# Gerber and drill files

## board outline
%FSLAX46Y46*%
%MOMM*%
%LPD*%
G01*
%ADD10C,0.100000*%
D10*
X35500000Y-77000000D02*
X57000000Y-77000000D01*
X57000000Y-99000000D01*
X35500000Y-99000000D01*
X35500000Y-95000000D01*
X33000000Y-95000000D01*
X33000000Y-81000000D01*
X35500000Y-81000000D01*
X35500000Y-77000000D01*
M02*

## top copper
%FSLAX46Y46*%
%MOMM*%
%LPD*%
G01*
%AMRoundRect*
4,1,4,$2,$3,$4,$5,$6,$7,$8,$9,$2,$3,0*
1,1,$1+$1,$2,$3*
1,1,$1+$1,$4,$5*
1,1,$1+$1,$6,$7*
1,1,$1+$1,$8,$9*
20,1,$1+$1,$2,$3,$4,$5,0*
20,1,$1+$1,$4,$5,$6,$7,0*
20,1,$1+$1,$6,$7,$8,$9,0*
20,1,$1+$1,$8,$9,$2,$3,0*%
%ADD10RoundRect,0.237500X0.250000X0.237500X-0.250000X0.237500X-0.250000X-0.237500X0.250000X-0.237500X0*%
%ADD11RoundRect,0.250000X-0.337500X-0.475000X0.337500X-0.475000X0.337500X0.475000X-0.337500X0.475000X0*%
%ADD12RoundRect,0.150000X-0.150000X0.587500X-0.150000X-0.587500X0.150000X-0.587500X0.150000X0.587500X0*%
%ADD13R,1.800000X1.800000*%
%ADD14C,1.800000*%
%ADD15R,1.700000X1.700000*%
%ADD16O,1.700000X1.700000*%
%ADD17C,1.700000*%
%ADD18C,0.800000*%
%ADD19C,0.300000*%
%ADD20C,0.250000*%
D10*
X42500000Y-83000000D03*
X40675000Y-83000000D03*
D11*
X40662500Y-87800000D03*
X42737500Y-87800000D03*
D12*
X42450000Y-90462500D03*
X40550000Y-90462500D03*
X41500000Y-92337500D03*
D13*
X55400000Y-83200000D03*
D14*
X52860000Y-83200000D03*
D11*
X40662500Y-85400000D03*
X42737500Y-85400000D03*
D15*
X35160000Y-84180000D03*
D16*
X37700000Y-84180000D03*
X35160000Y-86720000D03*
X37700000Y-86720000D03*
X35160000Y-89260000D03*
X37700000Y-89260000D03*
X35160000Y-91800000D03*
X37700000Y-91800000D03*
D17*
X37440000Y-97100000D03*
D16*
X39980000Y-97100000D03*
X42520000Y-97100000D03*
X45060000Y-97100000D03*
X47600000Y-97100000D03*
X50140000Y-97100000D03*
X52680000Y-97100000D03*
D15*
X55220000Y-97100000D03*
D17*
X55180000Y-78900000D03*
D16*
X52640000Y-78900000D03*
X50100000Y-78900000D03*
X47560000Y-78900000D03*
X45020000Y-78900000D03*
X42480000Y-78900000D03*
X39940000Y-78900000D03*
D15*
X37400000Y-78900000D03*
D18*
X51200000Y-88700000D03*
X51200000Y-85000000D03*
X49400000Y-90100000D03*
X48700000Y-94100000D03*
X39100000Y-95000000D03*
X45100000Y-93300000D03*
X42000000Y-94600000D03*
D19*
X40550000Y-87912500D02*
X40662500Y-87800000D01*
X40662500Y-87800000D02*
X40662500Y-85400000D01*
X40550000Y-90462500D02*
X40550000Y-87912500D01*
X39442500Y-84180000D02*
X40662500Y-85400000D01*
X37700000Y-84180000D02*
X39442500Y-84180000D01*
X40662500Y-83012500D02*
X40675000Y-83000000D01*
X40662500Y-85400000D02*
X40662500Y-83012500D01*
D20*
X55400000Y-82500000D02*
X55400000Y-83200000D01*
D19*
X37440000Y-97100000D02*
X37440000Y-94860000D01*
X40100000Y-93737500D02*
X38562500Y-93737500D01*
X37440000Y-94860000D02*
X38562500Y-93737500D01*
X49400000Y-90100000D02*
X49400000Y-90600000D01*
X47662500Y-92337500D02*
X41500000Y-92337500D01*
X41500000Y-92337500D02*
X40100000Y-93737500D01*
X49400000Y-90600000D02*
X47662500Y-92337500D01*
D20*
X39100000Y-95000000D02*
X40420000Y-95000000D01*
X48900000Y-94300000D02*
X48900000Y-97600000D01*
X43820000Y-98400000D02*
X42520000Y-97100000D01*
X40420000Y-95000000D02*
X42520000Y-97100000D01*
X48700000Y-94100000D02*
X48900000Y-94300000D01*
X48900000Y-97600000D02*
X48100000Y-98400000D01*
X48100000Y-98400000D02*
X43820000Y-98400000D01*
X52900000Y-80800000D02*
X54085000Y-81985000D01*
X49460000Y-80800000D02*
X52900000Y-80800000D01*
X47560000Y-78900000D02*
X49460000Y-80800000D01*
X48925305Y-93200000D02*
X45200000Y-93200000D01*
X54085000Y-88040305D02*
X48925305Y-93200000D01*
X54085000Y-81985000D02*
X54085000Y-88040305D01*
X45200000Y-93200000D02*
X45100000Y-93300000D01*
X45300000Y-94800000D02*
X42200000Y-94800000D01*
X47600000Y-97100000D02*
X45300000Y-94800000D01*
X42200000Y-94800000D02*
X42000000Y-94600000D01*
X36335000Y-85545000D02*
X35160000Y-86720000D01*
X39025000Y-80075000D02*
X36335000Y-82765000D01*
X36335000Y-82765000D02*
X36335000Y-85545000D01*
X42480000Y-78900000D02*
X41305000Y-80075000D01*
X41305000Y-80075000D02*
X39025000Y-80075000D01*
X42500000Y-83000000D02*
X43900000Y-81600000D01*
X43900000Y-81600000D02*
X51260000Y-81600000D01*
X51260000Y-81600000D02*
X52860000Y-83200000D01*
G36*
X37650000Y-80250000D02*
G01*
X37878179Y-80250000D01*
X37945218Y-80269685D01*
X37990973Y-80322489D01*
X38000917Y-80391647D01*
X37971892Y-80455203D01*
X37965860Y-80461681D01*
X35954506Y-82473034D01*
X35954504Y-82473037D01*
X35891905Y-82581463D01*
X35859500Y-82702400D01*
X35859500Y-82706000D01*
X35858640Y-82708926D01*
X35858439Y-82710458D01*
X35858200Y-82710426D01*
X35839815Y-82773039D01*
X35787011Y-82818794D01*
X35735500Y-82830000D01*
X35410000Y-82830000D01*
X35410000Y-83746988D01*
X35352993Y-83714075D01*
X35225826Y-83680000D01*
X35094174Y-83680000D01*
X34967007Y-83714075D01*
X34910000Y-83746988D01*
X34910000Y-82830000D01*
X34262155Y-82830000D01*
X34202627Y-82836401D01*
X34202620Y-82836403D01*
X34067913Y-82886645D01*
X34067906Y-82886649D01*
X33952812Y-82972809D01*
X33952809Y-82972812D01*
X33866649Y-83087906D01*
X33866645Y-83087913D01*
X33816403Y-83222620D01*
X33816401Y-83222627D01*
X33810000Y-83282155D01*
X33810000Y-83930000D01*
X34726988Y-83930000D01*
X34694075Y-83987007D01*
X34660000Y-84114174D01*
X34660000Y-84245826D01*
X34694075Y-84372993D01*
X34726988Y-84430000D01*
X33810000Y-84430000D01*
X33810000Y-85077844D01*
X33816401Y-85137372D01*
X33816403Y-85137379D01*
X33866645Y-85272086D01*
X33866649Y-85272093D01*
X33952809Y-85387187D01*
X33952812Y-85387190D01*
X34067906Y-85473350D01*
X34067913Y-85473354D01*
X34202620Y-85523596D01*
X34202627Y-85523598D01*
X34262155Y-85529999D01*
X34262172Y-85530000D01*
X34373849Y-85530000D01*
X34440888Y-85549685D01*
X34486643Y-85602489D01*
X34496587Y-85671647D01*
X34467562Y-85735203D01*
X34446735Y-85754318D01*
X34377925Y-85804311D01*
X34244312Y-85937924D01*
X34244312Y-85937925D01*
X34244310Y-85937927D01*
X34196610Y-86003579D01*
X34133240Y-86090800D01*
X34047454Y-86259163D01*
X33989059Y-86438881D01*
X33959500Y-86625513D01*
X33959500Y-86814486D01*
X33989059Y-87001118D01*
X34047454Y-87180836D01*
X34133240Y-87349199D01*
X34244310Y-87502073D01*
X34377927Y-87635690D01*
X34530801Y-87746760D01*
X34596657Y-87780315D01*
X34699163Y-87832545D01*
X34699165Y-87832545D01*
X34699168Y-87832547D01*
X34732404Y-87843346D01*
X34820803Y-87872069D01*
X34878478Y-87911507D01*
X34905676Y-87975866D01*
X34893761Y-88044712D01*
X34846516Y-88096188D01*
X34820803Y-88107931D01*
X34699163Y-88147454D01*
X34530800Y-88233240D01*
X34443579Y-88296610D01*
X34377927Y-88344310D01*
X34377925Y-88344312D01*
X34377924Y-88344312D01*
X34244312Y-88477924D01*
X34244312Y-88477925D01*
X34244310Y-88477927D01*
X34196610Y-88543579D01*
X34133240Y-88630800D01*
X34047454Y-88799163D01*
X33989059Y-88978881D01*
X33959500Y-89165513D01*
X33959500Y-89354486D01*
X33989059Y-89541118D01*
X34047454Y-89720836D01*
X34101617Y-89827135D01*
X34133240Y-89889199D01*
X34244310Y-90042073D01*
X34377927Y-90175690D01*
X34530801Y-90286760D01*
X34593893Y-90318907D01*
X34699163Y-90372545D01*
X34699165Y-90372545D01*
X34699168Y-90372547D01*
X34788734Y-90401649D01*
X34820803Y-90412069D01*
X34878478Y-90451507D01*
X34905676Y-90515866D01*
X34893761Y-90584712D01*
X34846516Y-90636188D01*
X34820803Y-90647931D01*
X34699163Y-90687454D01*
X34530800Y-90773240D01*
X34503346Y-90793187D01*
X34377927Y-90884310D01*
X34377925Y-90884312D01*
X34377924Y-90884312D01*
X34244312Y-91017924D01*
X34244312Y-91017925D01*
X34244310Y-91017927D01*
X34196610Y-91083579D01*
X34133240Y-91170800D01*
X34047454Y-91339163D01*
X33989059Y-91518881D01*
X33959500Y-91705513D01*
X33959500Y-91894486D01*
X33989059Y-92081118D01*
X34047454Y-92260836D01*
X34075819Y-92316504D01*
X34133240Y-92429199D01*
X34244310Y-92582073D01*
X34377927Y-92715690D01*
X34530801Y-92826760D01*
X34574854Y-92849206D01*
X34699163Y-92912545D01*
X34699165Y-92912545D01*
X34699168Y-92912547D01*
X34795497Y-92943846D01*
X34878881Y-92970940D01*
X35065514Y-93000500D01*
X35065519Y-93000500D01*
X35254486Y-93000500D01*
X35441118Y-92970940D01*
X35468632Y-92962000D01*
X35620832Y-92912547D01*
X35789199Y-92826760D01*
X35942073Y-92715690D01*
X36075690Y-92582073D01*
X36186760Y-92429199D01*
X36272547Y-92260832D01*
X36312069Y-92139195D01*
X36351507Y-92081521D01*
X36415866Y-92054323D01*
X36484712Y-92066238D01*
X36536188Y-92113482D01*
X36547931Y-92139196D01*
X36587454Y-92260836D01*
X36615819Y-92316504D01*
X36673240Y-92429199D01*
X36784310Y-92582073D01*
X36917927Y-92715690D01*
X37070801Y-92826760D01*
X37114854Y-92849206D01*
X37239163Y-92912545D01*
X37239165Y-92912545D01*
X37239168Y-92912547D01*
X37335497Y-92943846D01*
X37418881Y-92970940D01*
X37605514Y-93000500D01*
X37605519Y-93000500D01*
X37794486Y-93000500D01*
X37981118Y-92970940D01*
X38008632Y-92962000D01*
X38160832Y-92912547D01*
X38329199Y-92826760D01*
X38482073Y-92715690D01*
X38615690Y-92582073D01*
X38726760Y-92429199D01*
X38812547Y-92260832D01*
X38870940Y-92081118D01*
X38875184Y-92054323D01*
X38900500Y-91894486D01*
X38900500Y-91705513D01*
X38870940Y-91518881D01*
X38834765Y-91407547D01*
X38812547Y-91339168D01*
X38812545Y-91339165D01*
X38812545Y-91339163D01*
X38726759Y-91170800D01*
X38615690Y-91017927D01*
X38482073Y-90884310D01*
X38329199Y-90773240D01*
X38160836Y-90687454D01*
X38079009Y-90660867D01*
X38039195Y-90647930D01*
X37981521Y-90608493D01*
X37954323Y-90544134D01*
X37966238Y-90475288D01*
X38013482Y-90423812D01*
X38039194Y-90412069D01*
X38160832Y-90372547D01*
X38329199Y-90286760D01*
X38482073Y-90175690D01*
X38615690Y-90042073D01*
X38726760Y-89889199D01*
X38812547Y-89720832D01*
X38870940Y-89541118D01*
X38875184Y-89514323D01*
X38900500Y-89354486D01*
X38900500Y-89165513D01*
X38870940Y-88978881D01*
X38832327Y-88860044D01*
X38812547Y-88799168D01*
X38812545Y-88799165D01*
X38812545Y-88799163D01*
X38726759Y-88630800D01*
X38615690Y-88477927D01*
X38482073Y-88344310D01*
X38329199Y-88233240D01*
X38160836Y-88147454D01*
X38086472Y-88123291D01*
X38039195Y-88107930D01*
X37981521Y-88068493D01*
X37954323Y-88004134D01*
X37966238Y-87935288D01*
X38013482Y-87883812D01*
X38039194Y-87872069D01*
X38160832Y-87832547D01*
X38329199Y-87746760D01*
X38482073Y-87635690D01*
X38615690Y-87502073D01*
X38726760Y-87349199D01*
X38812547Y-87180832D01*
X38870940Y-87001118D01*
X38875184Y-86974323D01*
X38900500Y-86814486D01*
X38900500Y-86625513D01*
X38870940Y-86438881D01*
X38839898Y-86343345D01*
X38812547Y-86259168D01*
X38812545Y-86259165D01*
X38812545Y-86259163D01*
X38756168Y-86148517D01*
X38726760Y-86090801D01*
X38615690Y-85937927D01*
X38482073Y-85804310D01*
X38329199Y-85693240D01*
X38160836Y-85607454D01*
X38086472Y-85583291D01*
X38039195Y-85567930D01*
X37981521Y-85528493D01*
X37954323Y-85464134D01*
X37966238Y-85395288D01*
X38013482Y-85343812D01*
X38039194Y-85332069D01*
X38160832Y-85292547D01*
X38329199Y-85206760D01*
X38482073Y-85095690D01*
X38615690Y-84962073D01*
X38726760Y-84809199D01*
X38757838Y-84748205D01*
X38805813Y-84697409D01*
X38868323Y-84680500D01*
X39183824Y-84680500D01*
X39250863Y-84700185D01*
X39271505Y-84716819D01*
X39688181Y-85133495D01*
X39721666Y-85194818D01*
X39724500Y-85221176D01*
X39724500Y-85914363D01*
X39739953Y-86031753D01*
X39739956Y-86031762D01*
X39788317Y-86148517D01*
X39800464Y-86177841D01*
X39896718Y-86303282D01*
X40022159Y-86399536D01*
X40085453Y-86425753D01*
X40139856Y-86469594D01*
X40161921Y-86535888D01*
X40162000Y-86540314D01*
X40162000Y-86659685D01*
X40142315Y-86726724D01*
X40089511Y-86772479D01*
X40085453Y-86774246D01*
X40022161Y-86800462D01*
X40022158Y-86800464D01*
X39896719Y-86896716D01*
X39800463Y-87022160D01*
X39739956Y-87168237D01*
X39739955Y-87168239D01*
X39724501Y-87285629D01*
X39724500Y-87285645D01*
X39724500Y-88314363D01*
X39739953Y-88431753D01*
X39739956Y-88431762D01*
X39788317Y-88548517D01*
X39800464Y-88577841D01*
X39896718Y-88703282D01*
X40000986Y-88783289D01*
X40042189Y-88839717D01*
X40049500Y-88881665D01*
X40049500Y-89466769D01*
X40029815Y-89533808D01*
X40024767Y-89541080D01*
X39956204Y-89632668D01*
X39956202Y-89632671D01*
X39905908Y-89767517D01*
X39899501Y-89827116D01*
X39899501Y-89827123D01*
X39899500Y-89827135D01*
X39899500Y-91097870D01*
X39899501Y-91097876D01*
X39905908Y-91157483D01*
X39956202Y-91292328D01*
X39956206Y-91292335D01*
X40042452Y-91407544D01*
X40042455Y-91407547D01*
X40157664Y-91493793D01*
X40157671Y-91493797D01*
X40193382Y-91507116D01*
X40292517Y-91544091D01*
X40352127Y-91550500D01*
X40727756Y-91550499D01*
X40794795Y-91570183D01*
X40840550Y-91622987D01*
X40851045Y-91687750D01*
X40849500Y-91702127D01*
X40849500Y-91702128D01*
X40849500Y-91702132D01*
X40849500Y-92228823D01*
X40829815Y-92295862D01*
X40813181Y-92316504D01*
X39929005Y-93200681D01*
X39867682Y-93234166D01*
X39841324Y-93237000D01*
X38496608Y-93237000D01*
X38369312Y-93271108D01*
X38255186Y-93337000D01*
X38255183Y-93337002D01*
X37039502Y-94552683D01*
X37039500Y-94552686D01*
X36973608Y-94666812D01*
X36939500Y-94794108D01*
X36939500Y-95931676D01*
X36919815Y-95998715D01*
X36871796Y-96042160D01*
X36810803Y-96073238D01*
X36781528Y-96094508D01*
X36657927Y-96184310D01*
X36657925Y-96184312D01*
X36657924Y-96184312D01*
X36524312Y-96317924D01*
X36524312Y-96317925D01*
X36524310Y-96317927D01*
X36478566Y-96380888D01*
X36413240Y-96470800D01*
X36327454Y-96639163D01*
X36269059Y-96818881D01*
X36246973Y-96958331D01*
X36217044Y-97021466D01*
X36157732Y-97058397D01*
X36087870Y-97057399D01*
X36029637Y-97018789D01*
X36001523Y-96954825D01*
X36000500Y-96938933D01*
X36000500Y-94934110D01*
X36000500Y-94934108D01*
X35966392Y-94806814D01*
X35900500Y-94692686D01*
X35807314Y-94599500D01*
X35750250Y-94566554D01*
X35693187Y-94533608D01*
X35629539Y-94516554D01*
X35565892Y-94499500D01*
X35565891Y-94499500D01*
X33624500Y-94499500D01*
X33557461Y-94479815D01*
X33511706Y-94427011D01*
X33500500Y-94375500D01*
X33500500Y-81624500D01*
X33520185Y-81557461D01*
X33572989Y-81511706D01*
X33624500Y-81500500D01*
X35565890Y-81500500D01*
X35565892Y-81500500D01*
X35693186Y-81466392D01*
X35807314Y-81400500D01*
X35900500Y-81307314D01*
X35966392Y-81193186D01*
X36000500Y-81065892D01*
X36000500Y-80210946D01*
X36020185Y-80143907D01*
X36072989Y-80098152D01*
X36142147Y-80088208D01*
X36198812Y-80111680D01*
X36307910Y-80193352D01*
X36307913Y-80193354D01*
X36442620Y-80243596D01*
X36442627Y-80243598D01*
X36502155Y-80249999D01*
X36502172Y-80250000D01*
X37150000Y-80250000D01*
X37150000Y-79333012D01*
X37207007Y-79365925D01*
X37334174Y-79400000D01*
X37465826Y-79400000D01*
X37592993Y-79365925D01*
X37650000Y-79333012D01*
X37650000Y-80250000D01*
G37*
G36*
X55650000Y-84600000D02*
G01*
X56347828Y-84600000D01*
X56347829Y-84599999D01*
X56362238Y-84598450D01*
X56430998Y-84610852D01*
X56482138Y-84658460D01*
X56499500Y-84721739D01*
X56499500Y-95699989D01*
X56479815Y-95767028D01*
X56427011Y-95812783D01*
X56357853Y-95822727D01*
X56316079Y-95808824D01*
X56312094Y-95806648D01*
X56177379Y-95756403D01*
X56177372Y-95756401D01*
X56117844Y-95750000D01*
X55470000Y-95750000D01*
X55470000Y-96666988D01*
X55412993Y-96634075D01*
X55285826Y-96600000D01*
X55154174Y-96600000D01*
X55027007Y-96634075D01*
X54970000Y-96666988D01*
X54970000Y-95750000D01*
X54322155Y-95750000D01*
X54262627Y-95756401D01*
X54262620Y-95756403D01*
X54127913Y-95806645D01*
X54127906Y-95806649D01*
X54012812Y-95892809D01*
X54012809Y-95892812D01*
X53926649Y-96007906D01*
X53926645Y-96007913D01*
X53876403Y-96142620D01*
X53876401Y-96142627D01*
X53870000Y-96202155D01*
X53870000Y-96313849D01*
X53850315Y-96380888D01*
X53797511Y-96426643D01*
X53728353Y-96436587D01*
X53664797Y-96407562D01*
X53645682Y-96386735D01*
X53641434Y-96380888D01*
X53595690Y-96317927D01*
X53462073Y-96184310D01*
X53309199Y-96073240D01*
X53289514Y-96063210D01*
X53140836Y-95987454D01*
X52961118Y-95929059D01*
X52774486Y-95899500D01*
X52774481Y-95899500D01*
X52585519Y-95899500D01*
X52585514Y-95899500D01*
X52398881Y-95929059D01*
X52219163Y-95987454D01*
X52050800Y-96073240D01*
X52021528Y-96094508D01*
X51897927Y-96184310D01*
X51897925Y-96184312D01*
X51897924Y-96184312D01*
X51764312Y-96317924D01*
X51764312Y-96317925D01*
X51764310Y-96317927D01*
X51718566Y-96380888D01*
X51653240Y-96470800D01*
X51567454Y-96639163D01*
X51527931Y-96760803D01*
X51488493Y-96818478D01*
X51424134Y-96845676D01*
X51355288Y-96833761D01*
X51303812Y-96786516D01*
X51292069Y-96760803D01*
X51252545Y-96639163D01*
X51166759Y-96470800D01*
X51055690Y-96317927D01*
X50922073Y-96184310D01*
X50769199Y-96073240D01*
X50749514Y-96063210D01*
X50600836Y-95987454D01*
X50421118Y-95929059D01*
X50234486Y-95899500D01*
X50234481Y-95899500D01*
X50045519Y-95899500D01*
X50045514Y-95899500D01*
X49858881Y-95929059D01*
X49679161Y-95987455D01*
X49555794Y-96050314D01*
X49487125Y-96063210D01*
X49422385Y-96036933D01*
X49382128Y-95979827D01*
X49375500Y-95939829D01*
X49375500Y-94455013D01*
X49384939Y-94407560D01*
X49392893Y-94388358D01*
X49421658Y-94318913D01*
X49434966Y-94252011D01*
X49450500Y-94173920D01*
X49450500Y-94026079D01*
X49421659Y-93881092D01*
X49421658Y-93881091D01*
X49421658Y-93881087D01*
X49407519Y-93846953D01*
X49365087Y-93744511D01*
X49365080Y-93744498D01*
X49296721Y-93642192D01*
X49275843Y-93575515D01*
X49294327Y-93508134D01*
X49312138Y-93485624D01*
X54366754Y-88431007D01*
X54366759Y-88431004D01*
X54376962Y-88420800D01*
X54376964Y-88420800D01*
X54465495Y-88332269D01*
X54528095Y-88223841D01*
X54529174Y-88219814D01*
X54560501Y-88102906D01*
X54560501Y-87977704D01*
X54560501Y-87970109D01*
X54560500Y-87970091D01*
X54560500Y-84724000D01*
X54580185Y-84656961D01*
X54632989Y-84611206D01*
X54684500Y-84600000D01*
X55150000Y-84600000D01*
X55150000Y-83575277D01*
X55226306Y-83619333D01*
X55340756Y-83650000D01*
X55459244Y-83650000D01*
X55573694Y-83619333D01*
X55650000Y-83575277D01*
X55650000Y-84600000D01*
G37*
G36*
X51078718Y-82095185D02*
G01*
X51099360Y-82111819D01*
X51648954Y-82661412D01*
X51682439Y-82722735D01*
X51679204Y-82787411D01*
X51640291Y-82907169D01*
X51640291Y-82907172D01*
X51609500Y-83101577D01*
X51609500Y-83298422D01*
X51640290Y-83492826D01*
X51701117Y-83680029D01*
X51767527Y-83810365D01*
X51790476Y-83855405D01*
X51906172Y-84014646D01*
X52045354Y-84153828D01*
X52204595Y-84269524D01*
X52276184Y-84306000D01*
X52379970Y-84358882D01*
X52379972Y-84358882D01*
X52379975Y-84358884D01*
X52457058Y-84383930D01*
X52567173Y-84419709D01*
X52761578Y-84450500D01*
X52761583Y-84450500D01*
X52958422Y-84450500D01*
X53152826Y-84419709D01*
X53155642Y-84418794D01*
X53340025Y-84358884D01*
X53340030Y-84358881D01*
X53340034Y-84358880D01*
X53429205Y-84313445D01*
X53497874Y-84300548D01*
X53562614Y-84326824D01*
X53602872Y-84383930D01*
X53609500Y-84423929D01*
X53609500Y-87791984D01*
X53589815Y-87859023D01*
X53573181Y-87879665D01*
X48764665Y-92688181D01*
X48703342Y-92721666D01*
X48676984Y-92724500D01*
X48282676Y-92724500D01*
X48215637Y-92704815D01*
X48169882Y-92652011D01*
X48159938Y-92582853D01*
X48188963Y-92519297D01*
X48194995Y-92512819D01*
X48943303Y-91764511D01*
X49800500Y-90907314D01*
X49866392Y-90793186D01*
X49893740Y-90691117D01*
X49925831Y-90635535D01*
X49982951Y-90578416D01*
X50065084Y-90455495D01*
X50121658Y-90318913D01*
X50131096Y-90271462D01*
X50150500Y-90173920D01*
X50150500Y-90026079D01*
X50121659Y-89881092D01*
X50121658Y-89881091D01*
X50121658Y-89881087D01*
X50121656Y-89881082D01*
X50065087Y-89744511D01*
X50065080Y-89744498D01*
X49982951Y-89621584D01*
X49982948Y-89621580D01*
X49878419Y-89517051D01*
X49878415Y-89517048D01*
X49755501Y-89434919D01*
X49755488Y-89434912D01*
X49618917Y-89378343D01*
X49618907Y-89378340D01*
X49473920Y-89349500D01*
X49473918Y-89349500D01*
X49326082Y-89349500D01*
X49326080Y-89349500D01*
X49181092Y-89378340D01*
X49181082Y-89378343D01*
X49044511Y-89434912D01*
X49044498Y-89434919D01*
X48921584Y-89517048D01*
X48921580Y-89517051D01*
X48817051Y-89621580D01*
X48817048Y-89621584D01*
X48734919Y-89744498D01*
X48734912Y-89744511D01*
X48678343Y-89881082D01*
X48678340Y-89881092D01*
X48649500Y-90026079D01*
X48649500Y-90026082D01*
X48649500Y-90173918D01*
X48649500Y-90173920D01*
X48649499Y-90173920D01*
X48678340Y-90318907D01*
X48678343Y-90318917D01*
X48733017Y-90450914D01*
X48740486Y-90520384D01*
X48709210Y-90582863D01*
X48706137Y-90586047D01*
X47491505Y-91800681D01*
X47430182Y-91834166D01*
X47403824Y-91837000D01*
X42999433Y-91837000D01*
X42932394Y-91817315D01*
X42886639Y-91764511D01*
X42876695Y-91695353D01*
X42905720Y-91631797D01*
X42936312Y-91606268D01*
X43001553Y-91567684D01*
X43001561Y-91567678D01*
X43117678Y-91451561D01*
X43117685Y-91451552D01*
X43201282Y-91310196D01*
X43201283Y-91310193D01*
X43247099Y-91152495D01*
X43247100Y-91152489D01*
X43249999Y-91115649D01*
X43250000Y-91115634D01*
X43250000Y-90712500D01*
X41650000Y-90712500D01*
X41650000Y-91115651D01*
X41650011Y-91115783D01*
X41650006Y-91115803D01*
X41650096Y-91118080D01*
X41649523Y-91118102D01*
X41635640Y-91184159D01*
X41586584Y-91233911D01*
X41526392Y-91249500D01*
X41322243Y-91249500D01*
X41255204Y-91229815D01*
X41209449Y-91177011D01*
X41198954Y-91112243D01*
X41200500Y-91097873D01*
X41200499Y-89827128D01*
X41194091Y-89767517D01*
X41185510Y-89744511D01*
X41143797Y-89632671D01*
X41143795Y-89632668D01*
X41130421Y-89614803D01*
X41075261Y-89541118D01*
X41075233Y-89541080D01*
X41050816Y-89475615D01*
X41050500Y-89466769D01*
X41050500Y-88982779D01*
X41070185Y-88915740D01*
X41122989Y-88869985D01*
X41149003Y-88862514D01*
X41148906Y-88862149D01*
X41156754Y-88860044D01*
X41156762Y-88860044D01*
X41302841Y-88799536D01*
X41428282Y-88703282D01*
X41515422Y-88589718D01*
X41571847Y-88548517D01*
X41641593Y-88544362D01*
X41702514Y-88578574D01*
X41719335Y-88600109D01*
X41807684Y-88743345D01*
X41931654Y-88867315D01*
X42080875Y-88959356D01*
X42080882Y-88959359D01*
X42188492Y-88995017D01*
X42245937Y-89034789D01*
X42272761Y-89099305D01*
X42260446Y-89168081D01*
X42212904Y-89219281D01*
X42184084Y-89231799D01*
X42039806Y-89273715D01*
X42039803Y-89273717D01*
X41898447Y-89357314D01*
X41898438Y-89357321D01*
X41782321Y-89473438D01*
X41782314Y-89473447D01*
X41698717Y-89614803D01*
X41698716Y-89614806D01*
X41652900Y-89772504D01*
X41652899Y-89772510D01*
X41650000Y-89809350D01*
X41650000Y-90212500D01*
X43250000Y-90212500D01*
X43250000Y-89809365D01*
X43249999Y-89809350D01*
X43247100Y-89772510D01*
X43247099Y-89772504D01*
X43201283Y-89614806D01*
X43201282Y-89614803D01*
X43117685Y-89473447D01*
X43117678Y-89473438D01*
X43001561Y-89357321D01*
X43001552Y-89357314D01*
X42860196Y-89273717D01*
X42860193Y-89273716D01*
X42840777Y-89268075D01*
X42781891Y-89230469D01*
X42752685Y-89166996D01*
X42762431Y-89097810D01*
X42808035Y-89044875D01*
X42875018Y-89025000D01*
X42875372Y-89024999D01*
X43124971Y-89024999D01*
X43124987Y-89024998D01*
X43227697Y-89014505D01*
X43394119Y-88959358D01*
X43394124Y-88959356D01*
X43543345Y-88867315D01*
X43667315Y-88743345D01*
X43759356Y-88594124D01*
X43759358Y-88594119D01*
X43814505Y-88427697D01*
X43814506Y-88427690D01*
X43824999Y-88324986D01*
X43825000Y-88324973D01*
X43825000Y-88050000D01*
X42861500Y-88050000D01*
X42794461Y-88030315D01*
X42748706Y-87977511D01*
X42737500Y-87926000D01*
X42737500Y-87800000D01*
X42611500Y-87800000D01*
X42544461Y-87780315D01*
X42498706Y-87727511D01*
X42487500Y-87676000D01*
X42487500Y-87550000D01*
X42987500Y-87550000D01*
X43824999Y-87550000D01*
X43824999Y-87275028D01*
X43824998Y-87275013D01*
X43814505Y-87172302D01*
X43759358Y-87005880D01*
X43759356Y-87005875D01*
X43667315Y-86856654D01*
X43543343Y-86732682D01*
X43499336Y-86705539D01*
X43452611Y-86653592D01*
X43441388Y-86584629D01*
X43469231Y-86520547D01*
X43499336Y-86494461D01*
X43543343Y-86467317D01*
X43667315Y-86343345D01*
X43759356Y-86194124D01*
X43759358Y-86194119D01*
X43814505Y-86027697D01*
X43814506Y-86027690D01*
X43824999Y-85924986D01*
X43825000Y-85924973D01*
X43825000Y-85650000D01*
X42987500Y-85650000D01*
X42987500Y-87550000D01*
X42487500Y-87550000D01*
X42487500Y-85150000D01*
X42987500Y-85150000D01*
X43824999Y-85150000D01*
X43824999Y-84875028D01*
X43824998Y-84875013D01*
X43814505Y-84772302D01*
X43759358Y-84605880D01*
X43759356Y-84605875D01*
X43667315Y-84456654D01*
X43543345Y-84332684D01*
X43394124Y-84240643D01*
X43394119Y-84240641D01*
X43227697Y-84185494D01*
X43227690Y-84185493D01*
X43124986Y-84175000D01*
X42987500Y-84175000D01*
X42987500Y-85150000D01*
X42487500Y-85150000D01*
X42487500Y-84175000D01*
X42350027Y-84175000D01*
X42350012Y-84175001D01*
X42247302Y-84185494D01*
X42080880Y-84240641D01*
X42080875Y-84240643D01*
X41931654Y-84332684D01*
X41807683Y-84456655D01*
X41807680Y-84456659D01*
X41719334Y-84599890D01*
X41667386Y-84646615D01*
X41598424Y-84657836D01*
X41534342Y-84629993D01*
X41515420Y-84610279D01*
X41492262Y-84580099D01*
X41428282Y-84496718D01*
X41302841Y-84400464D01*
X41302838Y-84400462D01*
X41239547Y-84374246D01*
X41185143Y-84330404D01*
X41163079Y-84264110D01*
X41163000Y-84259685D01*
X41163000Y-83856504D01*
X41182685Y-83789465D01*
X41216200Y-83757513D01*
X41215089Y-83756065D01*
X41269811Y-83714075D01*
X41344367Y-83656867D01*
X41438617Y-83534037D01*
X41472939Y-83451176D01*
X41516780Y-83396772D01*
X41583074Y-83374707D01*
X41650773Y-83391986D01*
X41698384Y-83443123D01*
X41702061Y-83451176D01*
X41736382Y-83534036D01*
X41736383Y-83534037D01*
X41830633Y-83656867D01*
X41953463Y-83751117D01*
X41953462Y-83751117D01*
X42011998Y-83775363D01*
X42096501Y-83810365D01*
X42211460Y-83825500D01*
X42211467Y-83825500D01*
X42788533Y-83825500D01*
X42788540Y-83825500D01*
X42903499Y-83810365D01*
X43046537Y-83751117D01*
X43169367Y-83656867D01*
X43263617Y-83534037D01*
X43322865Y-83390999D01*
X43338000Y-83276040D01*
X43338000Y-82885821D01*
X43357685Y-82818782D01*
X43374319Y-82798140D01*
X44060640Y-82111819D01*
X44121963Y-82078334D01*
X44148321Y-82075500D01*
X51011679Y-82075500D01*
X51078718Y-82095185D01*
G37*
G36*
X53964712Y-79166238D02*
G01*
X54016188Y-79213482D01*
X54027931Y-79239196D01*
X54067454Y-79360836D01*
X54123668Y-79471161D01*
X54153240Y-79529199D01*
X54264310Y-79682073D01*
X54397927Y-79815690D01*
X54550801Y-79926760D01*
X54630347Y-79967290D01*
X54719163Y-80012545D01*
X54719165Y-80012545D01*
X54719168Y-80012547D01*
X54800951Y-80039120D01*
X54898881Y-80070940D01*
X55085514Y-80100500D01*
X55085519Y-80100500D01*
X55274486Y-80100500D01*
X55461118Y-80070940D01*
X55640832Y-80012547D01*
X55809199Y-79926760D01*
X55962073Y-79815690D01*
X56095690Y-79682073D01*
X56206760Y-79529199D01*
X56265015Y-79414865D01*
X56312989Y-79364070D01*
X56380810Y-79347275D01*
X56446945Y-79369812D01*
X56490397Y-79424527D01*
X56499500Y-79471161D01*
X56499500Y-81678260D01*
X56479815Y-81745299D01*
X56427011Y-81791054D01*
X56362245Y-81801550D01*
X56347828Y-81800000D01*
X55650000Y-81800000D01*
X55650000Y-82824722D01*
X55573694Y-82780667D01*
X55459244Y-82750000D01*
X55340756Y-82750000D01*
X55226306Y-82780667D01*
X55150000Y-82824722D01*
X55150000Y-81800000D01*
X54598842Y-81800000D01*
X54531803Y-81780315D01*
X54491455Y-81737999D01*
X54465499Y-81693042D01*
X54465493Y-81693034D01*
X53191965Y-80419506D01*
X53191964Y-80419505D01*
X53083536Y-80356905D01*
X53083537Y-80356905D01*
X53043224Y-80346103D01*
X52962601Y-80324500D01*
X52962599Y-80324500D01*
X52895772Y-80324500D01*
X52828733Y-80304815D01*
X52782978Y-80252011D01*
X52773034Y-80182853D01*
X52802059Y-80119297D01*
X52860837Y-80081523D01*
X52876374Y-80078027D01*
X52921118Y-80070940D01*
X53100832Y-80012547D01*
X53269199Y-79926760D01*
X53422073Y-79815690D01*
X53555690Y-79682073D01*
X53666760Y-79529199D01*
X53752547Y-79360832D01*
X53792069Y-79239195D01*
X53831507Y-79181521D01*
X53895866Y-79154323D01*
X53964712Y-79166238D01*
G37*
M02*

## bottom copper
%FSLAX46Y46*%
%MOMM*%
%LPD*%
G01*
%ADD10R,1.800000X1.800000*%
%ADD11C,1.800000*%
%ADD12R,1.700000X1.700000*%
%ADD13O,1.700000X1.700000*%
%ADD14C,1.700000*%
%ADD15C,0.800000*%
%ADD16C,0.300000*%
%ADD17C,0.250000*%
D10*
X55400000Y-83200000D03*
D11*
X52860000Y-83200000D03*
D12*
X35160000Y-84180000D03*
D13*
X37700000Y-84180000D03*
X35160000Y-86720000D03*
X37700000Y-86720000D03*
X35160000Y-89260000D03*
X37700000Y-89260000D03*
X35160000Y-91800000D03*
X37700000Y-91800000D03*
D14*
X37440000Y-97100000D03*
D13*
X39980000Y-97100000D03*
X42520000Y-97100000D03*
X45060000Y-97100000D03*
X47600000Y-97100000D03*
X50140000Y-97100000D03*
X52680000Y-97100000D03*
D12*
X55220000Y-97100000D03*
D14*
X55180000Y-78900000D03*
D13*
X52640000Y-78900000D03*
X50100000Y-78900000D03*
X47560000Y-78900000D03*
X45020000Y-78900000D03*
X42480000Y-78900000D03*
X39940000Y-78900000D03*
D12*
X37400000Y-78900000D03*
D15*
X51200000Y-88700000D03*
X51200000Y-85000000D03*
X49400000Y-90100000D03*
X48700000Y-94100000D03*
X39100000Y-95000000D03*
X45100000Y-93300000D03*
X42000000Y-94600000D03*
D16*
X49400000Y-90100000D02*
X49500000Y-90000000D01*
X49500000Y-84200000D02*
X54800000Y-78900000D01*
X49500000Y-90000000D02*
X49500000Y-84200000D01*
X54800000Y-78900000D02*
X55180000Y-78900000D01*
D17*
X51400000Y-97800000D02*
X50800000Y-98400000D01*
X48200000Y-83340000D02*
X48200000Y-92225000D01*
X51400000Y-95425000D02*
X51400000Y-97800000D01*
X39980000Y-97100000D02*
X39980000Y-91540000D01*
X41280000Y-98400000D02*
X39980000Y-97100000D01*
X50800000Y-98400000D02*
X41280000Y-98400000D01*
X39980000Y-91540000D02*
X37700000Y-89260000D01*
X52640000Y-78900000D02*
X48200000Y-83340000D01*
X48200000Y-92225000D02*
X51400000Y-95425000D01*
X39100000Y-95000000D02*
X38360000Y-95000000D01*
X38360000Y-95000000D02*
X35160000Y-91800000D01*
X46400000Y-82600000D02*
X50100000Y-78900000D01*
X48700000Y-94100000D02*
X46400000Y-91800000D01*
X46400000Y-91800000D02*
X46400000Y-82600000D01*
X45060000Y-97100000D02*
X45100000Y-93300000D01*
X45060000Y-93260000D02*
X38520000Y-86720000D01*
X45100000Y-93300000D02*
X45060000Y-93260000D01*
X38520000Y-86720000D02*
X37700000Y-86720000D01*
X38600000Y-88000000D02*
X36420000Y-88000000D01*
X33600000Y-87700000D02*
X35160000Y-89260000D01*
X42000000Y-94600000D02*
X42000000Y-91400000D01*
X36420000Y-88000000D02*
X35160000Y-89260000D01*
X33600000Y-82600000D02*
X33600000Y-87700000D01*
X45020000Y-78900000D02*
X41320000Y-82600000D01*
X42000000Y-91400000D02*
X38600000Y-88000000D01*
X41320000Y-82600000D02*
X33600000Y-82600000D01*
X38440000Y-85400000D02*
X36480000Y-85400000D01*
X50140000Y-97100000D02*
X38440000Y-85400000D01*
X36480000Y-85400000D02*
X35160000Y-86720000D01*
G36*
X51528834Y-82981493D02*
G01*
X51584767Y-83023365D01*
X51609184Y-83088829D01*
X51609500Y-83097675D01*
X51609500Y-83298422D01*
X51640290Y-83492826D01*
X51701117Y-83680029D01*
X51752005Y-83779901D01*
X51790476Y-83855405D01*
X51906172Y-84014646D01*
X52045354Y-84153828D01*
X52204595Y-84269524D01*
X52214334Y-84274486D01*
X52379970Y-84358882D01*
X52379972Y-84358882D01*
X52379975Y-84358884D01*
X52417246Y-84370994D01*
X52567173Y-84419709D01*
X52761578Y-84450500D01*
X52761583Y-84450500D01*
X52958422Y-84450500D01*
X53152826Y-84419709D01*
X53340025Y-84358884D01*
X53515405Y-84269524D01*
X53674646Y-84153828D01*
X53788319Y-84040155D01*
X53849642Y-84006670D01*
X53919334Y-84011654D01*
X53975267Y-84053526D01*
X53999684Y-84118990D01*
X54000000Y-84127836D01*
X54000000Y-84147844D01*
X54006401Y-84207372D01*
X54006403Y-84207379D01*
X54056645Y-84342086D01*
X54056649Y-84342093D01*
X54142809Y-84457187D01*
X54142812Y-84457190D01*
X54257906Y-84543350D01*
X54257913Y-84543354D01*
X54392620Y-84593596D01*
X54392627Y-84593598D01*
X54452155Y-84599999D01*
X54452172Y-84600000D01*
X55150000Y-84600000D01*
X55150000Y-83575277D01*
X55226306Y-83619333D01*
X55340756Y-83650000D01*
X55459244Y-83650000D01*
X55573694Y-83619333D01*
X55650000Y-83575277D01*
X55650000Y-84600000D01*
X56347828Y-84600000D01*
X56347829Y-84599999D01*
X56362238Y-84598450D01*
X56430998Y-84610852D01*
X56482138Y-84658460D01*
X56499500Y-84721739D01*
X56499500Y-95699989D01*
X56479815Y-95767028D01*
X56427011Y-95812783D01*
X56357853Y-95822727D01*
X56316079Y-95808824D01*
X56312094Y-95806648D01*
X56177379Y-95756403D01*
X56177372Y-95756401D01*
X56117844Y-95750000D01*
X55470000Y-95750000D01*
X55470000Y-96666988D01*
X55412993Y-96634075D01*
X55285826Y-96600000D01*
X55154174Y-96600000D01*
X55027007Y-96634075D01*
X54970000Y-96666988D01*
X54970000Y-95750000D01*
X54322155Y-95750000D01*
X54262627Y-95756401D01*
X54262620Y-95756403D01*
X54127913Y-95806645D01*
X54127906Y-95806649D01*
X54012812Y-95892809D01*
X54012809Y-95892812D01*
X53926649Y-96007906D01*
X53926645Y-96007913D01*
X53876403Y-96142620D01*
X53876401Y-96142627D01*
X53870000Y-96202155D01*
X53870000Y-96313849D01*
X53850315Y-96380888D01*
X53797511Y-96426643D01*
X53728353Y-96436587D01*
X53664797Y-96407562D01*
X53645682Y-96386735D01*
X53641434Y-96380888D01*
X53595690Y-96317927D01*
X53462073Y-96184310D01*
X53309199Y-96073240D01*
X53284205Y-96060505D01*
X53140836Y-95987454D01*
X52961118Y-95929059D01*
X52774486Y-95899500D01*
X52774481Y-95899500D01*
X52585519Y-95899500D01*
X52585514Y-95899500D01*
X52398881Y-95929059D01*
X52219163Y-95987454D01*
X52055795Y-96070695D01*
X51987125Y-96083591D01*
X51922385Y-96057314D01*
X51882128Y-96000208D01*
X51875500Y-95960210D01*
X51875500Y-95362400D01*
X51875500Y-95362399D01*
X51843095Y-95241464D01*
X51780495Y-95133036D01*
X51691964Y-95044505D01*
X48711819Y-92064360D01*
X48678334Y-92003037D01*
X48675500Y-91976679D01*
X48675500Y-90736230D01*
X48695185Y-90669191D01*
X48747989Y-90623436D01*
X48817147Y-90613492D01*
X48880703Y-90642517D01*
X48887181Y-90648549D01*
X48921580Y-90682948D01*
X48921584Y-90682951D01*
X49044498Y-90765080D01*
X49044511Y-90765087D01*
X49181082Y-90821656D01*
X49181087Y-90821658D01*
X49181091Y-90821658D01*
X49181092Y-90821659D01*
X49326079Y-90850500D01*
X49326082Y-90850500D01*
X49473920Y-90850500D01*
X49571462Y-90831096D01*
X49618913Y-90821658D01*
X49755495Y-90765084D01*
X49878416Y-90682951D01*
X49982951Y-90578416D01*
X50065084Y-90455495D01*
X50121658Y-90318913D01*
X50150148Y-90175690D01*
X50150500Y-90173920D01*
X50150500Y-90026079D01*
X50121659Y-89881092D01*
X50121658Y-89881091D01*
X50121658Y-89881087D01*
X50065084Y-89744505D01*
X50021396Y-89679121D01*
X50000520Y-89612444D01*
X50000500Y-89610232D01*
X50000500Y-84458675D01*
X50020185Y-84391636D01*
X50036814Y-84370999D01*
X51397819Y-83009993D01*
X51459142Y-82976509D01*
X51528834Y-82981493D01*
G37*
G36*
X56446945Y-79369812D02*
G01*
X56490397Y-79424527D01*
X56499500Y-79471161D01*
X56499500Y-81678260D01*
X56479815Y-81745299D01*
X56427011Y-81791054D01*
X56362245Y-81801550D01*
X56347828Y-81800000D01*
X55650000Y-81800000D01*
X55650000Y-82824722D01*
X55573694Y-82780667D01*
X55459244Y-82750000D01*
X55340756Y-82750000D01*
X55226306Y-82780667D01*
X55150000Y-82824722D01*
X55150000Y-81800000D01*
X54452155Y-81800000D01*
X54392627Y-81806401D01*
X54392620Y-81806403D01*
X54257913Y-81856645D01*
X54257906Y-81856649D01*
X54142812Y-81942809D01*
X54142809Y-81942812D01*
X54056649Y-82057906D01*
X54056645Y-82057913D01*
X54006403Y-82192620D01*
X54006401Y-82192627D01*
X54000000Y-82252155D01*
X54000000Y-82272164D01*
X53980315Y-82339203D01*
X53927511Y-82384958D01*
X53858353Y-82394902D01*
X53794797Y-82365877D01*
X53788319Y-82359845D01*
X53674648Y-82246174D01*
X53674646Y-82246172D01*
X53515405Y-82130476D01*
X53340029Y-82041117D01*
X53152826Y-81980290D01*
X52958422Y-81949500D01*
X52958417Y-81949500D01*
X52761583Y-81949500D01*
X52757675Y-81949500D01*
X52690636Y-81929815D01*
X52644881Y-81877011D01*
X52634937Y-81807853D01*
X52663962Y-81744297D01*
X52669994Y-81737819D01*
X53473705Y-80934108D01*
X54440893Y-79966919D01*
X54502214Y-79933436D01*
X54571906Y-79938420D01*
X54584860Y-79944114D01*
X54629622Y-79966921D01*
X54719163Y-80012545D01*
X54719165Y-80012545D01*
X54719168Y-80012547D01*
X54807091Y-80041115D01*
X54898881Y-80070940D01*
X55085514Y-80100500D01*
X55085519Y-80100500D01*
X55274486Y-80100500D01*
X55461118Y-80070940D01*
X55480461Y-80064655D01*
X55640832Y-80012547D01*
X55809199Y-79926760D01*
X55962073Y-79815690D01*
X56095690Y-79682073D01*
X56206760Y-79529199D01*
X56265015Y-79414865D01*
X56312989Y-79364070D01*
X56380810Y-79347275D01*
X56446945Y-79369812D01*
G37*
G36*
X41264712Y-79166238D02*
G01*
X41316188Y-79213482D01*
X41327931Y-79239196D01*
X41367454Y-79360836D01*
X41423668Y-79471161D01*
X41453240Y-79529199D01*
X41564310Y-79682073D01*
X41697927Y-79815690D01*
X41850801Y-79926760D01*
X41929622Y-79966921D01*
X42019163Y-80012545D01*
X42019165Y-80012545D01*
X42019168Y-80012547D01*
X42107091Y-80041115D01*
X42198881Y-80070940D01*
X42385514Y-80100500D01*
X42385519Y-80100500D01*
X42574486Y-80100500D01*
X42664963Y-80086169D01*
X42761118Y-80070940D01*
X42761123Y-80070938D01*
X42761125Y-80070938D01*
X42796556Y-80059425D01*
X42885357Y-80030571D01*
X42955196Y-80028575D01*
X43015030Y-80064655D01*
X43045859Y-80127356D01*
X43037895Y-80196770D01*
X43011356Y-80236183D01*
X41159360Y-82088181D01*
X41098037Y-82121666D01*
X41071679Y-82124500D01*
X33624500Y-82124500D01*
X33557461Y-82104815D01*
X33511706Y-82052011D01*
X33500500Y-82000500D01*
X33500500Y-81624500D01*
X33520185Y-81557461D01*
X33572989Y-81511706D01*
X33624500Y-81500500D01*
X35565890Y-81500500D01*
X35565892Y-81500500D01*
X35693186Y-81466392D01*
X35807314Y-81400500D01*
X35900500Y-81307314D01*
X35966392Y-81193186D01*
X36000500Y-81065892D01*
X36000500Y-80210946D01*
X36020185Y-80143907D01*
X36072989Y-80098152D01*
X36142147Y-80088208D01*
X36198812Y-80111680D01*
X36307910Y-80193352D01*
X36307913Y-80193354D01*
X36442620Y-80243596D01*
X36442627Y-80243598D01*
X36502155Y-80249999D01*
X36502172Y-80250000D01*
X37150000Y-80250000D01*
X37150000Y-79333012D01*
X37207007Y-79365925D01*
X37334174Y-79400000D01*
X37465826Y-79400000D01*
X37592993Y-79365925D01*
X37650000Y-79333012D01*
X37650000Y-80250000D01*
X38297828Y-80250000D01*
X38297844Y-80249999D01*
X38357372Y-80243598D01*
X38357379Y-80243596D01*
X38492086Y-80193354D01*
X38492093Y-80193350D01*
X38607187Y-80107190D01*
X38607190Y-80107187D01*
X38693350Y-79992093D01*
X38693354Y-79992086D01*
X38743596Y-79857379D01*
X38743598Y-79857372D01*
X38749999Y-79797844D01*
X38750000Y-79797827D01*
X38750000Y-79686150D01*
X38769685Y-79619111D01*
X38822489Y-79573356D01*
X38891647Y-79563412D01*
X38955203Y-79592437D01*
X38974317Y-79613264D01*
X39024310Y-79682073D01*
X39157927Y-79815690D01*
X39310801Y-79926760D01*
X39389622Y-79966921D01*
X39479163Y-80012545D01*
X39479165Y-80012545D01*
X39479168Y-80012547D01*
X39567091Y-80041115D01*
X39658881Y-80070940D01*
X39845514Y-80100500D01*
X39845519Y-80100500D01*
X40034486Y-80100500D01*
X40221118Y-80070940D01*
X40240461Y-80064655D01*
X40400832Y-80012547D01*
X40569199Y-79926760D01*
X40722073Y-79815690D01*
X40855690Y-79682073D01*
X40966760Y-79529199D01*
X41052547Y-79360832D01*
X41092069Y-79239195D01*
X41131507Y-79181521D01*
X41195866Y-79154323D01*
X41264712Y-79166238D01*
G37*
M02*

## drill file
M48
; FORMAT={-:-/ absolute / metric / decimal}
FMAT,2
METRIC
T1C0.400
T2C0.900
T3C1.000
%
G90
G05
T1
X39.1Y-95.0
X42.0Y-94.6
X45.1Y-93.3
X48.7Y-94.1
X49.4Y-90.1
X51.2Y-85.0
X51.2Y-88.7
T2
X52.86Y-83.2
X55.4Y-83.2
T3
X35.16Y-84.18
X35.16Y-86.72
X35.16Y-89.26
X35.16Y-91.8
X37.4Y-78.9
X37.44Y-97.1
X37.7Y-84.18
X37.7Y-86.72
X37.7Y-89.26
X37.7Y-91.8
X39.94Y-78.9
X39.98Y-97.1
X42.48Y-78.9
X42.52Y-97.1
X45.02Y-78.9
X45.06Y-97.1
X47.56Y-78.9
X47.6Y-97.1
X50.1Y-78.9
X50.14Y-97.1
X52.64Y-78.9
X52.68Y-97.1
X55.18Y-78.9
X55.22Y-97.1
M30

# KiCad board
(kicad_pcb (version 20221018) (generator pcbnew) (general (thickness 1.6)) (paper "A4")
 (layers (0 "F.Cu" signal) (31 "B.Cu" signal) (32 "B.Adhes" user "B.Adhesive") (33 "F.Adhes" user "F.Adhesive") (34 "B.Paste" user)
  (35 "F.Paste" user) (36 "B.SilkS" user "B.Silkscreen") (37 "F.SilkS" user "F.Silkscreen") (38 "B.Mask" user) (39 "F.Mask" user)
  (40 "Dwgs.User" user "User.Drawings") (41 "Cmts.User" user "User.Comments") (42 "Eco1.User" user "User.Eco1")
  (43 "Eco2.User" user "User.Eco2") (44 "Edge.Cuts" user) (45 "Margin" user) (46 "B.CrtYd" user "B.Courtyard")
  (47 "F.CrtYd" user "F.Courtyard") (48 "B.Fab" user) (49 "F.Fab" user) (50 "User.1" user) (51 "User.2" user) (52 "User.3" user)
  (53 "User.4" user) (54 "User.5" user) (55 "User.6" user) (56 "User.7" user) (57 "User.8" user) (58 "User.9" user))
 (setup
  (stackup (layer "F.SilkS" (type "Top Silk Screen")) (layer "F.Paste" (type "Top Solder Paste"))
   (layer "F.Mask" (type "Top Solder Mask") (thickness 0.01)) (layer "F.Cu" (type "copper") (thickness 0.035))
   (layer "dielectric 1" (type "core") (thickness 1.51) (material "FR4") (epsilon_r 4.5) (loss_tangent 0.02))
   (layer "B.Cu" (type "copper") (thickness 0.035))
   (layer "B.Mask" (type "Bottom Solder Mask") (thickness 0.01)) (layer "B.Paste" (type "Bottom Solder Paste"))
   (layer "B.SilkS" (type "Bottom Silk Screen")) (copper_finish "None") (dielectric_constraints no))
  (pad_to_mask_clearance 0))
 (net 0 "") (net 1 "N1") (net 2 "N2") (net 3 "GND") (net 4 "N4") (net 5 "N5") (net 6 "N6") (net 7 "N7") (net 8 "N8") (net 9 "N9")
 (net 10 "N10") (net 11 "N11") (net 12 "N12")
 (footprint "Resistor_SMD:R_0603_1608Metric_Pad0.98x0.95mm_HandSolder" (layer "F.Cu") (at 41.5875 83 180)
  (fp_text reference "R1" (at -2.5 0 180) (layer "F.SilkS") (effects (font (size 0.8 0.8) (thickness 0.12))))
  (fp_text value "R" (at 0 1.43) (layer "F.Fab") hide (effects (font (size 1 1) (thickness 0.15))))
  (pad "1" smd roundrect (at -0.9125 0 180) (size 0.975 0.95) (layers "F.Cu" "F.Paste" "F.Mask") (roundrect_rratio 0.25) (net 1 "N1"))
  (pad "2" smd roundrect (at 0.9125 0 180) (size 0.975 0.95) (layers "F.Cu" "F.Paste" "F.Mask") (roundrect_rratio 0.25) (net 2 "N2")))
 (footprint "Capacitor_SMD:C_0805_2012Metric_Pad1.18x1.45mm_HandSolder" (layer "F.Cu") (at 41.7 87.8)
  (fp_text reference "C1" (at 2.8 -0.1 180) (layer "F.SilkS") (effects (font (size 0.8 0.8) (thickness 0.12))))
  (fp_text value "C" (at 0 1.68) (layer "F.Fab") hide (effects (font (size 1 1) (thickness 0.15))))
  (pad "1" smd roundrect (at -1.0375 0) (size 1.175 1.45) (layers "F.Cu" "F.Paste" "F.Mask") (roundrect_rratio 0.2127659574) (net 2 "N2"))
  (pad "2" smd roundrect (at 1.0375 0) (size 1.175 1.45) (layers "F.Cu" "F.Paste" "F.Mask") (roundrect_rratio 0.2127659574) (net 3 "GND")))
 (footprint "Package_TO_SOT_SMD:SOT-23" (layer "F.Cu") (at 41.5 91.4 -90)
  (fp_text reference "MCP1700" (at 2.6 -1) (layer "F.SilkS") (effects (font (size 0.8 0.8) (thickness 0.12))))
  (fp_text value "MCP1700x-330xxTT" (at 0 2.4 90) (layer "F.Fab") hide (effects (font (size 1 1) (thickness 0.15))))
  (pad "1" smd roundrect (at -0.9375 -0.95 270) (size 1.475 0.6) (layers "F.Cu" "F.Paste" "F.Mask") (roundrect_rratio 0.25) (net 3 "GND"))
  (pad "2" smd roundrect (at -0.9375 0.95 270) (size 1.475 0.6) (layers "F.Cu" "F.Paste" "F.Mask") (roundrect_rratio 0.25) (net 2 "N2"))
  (pad "3" smd roundrect (at 0.9375 0 270) (size 1.475 0.6) (layers "F.Cu" "F.Paste" "F.Mask") (roundrect_rratio 0.25) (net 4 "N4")))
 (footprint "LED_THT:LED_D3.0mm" (layer "F.Cu") (at 55.4 83.2 180)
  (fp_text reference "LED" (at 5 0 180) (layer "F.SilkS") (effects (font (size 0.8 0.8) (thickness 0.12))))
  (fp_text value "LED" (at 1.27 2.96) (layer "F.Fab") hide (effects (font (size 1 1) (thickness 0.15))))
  (pad "1" thru_hole rect (at 0 0 180) (size 1.8 1.8) (drill 0.9) (layers "*.Cu" "*.Mask") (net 3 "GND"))
  (pad "2" thru_hole circle (at 2.54 0 180) (size 1.8 1.8) (drill 0.9) (layers "*.Cu" "*.Mask") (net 1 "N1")))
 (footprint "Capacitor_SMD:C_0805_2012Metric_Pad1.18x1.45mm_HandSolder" (layer "F.Cu") (at 41.7 85.4)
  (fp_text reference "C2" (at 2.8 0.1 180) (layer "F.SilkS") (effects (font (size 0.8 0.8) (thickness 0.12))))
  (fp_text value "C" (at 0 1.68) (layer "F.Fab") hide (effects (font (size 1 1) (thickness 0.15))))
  (pad "1" smd roundrect (at -1.0375 0) (size 1.175 1.45) (layers "F.Cu" "F.Paste" "F.Mask") (roundrect_rratio 0.2127659574) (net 2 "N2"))
  (pad "2" smd roundrect (at 1.0375 0) (size 1.175 1.45) (layers "F.Cu" "F.Paste" "F.Mask") (roundrect_rratio 0.2127659574) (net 3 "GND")))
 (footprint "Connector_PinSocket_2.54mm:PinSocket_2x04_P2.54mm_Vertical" (layer "B.Cu") (at 35.16 84.18 180)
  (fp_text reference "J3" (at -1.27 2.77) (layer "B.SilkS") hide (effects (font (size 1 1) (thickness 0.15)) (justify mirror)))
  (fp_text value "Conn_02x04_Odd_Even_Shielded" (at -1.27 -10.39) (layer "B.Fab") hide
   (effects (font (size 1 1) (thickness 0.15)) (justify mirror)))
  (pad "1" thru_hole rect (at 0 0 180) (size 1.7 1.7) (drill 1) (layers "*.Cu" "*.Mask") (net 3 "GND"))
  (pad "2" thru_hole oval (at -2.54 0 180) (size 1.7 1.7) (drill 1) (layers "*.Cu" "*.Mask") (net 2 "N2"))
  (pad "3" thru_hole oval (at 0 -2.54 180) (size 1.7 1.7) (drill 1) (layers "*.Cu" "*.Mask") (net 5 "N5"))
  (pad "4" thru_hole oval (at -2.54 -2.54 180) (size 1.7 1.7) (drill 1) (layers "*.Cu" "*.Mask") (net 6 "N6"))
  (pad "5" thru_hole oval (at 0 -5.08 180) (size 1.7 1.7) (drill 1) (layers "*.Cu" "*.Mask") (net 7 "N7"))
  (pad "6" thru_hole oval (at -2.54 -5.08 180) (size 1.7 1.7) (drill 1) (layers "*.Cu" "*.Mask") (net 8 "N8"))
  (pad "7" thru_hole oval (at 0 -7.62 180) (size 1.7 1.7) (drill 1) (layers "*.Cu" "*.Mask") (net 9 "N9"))
  (pad "8" thru_hole oval (at -2.54 -7.62 180) (size 1.7 1.7) (drill 1) (layers "*.Cu" "*.Mask") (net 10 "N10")))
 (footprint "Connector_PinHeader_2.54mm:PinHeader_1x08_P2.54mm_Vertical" (layer "B.Cu") (at 37.44 97.1 -90)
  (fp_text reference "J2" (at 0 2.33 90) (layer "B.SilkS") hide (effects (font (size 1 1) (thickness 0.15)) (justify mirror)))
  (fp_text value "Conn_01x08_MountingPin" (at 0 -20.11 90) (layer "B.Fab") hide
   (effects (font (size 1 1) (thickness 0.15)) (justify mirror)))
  (pad "1" thru_hole circle (at 0 0 270) (size 1.7 1.7) (drill 1) (layers "*.Cu" "*.Mask") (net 4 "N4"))
  (pad "2" thru_hole oval (at 0 -2.54 270) (size 1.7 1.7) (drill 1) (layers "*.Cu" "*.Mask") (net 8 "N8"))
  (pad "3" thru_hole oval (at 0 -5.08 270) (size 1.7 1.7) (drill 1) (layers "*.Cu" "*.Mask") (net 9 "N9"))
  (pad "4" thru_hole oval (at 0 -7.62 270) (size 1.7 1.7) (drill 1) (layers "*.Cu" "*.Mask") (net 6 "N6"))
  (pad "5" thru_hole oval (at 0 -10.16 270) (size 1.7 1.7) (drill 1) (layers "*.Cu" "*.Mask") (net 7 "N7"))
  (pad "6" thru_hole oval (at 0 -12.7 270) (size 1.7 1.7) (drill 1) (layers "*.Cu" "*.Mask") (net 5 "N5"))
  (pad "7" thru_hole oval (at 0 -15.24 270) (size 1.7 1.7) (drill 1) (layers "*.Cu" "*.Mask") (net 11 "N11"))
  (pad "8" thru_hole rect (at 0 -17.78 270) (size 1.7 1.7) (drill 1) (layers "*.Cu" "*.Mask") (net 3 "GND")))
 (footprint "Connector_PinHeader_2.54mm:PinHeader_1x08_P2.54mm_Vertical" (layer "B.Cu") (at 55.18 78.9 90)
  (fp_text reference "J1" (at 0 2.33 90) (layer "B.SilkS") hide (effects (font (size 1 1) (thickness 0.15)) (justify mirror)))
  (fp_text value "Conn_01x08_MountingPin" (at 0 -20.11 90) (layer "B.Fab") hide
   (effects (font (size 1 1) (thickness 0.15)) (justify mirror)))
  (pad "1" thru_hole circle (at 0 0 90) (size 1.7 1.7) (drill 1) (layers "*.Cu" "*.Mask") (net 4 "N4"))
  (pad "2" thru_hole oval (at 0 -2.54 90) (size 1.7 1.7) (drill 1) (layers "*.Cu" "*.Mask") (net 8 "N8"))
  (pad "3" thru_hole oval (at 0 -5.08 90) (size 1.7 1.7) (drill 1) (layers "*.Cu" "*.Mask") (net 9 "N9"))
  (pad "4" thru_hole oval (at 0 -7.62 90) (size 1.7 1.7) (drill 1) (layers "*.Cu" "*.Mask") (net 6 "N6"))
  (pad "5" thru_hole oval (at 0 -10.16 90) (size 1.7 1.7) (drill 1) (layers "*.Cu" "*.Mask") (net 7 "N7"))
  (pad "6" thru_hole oval (at 0 -12.7 90) (size 1.7 1.7) (drill 1) (layers "*.Cu" "*.Mask") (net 5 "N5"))
  (pad "7" thru_hole oval (at 0 -15.24 90) (size 1.7 1.7) (drill 1) (layers "*.Cu" "*.Mask") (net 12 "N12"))
  (pad "8" thru_hole rect (at 0 -17.78 90) (size 1.7 1.7) (drill 1) (layers "*.Cu" "*.Mask") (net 3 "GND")))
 (gr_poly
  (pts (xy 35.5 77) (xy 57 77) (xy 57 99) (xy 35.5 99) (xy 35.5 95) (xy 33 95) (xy 33 81) (xy 35.5 81)) (stroke (width 0.1) (type solid))
  (fill none) (layer "Edge.Cuts"))
 (segment (start 40.55 87.9125) (end 40.6625 87.8) (width 0.3) (layer "F.Cu") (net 2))
 (segment (start 40.6625 87.8) (end 40.6625 85.4) (width 0.3) (layer "F.Cu") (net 2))
 (segment (start 40.55 90.4625) (end 40.55 87.9125) (width 0.3) (layer "F.Cu") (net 2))
 (segment (start 39.4425 84.18) (end 40.6625 85.4) (width 0.3) (layer "F.Cu") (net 2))
 (segment (start 37.7 84.18) (end 39.4425 84.18) (width 0.3) (layer "F.Cu") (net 2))
 (segment (start 40.6625 83.0125) (end 40.675 83) (width 0.3) (layer "F.Cu") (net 2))
 (segment (start 40.6625 85.4) (end 40.6625 83.0125) (width 0.3) (layer "F.Cu") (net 2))
 (segment (start 55.4 82.5) (end 55.4 83.2) (width 0.25) (layer "F.Cu") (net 3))
 (via (at 51.2 88.7) (size 0.8) (drill 0.4) (layers "F.Cu" "B.Cu") (free) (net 3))
 (via (at 51.2 85) (size 0.8) (drill 0.4) (layers "F.Cu" "B.Cu") (free) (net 3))
 (segment (start 37.44 97.1) (end 37.44 94.86) (width 0.3) (layer "F.Cu") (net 4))
 (segment (start 40.1 93.7375) (end 38.5625 93.7375) (width 0.3) (layer "F.Cu") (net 4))
 (segment (start 37.44 94.86) (end 38.5625 93.7375) (width 0.3) (layer "F.Cu") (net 4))
 (segment (start 49.4 90.1) (end 49.4 90.6) (width 0.3) (layer "F.Cu") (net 4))
 (segment (start 47.6625 92.3375) (end 41.5 92.3375) (width 0.3) (layer "F.Cu") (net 4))
 (segment (start 41.5 92.3375) (end 40.1 93.7375) (width 0.3) (layer "F.Cu") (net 4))
 (segment (start 49.4 90.6) (end 47.6625 92.3375) (width 0.3) (layer "F.Cu") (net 4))
 (via (at 49.4 90.1) (size 0.8) (drill 0.4) (layers "F.Cu" "B.Cu") (free) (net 4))
 (segment (start 49.4 90.1) (end 49.5 90) (width 0.3) (layer "B.Cu") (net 4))
 (segment (start 49.5 84.2) (end 54.8 78.9) (width 0.3) (layer "B.Cu") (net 4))
 (segment (start 49.5 90) (end 49.5 84.2) (width 0.3) (layer "B.Cu") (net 4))
 (segment (start 54.8 78.9) (end 55.18 78.9) (width 0.3) (layer "B.Cu") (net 4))
 (segment (start 51.4 97.8) (end 50.8 98.4) (width 0.25) (layer "B.Cu") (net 8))
 (segment (start 48.2 83.34) (end 48.2 92.225) (width 0.25) (layer "B.Cu") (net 8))
 (segment (start 51.4 95.425) (end 51.4 97.8) (width 0.25) (layer "B.Cu") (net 8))
 (segment (start 39.98 97.1) (end 39.98 91.54) (width 0.25) (layer "B.Cu") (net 8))
 (segment (start 41.28 98.4) (end 39.98 97.1) (width 0.25) (layer "B.Cu") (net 8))
 (segment (start 50.8 98.4) (end 41.28 98.4) (width 0.25) (layer "B.Cu") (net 8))
 (segment (start 39.98 91.54) (end 37.7 89.26) (width 0.25) (layer "B.Cu") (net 8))
 (segment (start 52.64 78.9) (end 48.2 83.34) (width 0.25) (layer "B.Cu") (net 8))
 (segment (start 48.2 92.225) (end 51.4 95.425) (width 0.25) (layer "B.Cu") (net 8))
 (segment (start 39.1 95) (end 40.42 95) (width 0.25) (layer "F.Cu") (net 9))
 (segment (start 48.9 94.3) (end 48.9 97.6) (width 0.25) (layer "F.Cu") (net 9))
 (segment (start 43.82 98.4) (end 42.52 97.1) (width 0.25) (layer "F.Cu") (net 9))
 (segment (start 40.42 95) (end 42.52 97.1) (width 0.25) (layer "F.Cu") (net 9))
 (segment (start 48.7 94.1) (end 48.9 94.3) (width 0.25) (layer "F.Cu") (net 9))
 (segment (start 48.9 97.6) (end 48.1 98.4) (width 0.25) (layer "F.Cu") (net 9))
 (segment (start 48.1 98.4) (end 43.82 98.4) (width 0.25) (layer "F.Cu") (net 9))
 (via (at 48.7 94.1) (size 0.8) (drill 0.4) (layers "F.Cu" "B.Cu") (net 9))
 (via (at 39.1 95) (size 0.8) (drill 0.4) (layers "F.Cu" "B.Cu") (free) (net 9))
 (segment (start 39.1 95) (end 38.36 95) (width 0.25) (layer "B.Cu") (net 9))
 (segment (start 38.36 95) (end 35.16 91.8) (width 0.25) (layer "B.Cu") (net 9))
 (segment (start 46.4 82.6) (end 50.1 78.9) (width 0.25) (layer "B.Cu") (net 9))
 (segment (start 48.7 94.1) (end 46.4 91.8) (width 0.25) (layer "B.Cu") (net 9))
 (segment (start 46.4 91.8) (end 46.4 82.6) (width 0.25) (layer "B.Cu") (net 9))
 (segment (start 52.9 80.8) (end 54.085 81.985) (width 0.25) (layer "F.Cu") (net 6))
 (segment (start 49.46 80.8) (end 52.9 80.8) (width 0.25) (layer "F.Cu") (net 6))
 (segment (start 47.56 78.9) (end 49.46 80.8) (width 0.25) (layer "F.Cu") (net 6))
 (segment (start 48.925305 93.2) (end 45.2 93.2) (width 0.25) (layer "F.Cu") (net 6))
 (segment (start 54.085 88.040305) (end 48.925305 93.2) (width 0.25) (layer "F.Cu") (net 6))
 (segment (start 54.085 81.985) (end 54.085 88.040305) (width 0.25) (layer "F.Cu") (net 6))
 (segment (start 45.2 93.2) (end 45.1 93.3) (width 0.25) (layer "F.Cu") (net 6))
 (via (at 45.1 93.3) (size 0.8) (drill 0.4) (layers "F.Cu" "B.Cu") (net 6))
 (segment (start 45.06 97.1) (end 45.1 93.3) (width 0.25) (layer "B.Cu") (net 6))
 (segment (start 45.06 93.26) (end 38.52 86.72) (width 0.25) (layer "B.Cu") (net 6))
 (segment (start 45.1 93.3) (end 45.06 93.26) (width 0.25) (layer "B.Cu") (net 6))
 (segment (start 38.52 86.72) (end 37.7 86.72) (width 0.25) (layer "B.Cu") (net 6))
 (segment (start 45.3 94.8) (end 42.2 94.8) (width 0.25) (layer "F.Cu") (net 7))
 (segment (start 47.6 97.1) (end 45.3 94.8) (width 0.25) (layer "F.Cu") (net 7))
 (segment (start 42.2 94.8) (end 42 94.6) (width 0.25) (layer "F.Cu") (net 7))
 (via (at 42 94.6) (size 0.8) (drill 0.4) (layers "F.Cu" "B.Cu") (free) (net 7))
 (segment (start 38.6 88) (end 36.42 88) (width 0.25) (layer "B.Cu") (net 7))
 (segment (start 33.6 87.7) (end 35.16 89.26) (width 0.25) (layer "B.Cu") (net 7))
 (segment (start 42 94.6) (end 42 91.4) (width 0.25) (layer "B.Cu") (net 7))
 (segment (start 36.42 88) (end 35.16 89.26) (width 0.25) (layer "B.Cu") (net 7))
 (segment (start 33.6 82.6) (end 33.6 87.7) (width 0.25) (layer "B.Cu") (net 7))
 (segment (start 45.02 78.9) (end 41.32 82.6) (width 0.25) (layer "B.Cu") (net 7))
 (segment (start 42 91.4) (end 38.6 88) (width 0.25) (layer "B.Cu") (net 7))
 (segment (start 41.32 82.6) (end 33.6 82.6) (width 0.25) (layer "B.Cu") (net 7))
 (segment (start 36.335 85.545) (end 35.16 86.72) (width 0.25) (layer "F.Cu") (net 5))
 (segment (start 39.025 80.075) (end 36.335 82.765) (width 0.25) (layer "F.Cu") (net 5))
 (segment (start 36.335 82.765) (end 36.335 85.545) (width 0.25) (layer "F.Cu") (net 5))
 (segment (start 42.48 78.9) (end 41.305 80.075) (width 0.25) (layer "F.Cu") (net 5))
 (segment (start 41.305 80.075) (end 39.025 80.075) (width 0.25) (layer "F.Cu") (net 5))
 (segment (start 38.44 85.4) (end 36.48 85.4) (width 0.25) (layer "B.Cu") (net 5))
 (segment (start 50.14 97.1) (end 38.44 85.4) (width 0.25) (layer "B.Cu") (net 5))
 (segment (start 36.48 85.4) (end 35.16 86.72) (width 0.25) (layer "B.Cu") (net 5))
 (segment (start 42.5 83) (end 43.9 81.6) (width 0.25) (layer "F.Cu") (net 1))
 (segment (start 43.9 81.6) (end 51.26 81.6) (width 0.25) (layer "F.Cu") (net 1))
 (segment (start 51.26 81.6) (end 52.86 83.2) (width 0.25) (layer "F.Cu") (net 1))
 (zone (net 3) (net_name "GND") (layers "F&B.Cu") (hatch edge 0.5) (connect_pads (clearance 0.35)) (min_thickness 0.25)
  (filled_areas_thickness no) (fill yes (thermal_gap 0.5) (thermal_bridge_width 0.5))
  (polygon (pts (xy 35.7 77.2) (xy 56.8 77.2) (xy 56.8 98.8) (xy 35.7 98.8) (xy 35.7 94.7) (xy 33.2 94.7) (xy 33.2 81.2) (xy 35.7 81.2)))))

